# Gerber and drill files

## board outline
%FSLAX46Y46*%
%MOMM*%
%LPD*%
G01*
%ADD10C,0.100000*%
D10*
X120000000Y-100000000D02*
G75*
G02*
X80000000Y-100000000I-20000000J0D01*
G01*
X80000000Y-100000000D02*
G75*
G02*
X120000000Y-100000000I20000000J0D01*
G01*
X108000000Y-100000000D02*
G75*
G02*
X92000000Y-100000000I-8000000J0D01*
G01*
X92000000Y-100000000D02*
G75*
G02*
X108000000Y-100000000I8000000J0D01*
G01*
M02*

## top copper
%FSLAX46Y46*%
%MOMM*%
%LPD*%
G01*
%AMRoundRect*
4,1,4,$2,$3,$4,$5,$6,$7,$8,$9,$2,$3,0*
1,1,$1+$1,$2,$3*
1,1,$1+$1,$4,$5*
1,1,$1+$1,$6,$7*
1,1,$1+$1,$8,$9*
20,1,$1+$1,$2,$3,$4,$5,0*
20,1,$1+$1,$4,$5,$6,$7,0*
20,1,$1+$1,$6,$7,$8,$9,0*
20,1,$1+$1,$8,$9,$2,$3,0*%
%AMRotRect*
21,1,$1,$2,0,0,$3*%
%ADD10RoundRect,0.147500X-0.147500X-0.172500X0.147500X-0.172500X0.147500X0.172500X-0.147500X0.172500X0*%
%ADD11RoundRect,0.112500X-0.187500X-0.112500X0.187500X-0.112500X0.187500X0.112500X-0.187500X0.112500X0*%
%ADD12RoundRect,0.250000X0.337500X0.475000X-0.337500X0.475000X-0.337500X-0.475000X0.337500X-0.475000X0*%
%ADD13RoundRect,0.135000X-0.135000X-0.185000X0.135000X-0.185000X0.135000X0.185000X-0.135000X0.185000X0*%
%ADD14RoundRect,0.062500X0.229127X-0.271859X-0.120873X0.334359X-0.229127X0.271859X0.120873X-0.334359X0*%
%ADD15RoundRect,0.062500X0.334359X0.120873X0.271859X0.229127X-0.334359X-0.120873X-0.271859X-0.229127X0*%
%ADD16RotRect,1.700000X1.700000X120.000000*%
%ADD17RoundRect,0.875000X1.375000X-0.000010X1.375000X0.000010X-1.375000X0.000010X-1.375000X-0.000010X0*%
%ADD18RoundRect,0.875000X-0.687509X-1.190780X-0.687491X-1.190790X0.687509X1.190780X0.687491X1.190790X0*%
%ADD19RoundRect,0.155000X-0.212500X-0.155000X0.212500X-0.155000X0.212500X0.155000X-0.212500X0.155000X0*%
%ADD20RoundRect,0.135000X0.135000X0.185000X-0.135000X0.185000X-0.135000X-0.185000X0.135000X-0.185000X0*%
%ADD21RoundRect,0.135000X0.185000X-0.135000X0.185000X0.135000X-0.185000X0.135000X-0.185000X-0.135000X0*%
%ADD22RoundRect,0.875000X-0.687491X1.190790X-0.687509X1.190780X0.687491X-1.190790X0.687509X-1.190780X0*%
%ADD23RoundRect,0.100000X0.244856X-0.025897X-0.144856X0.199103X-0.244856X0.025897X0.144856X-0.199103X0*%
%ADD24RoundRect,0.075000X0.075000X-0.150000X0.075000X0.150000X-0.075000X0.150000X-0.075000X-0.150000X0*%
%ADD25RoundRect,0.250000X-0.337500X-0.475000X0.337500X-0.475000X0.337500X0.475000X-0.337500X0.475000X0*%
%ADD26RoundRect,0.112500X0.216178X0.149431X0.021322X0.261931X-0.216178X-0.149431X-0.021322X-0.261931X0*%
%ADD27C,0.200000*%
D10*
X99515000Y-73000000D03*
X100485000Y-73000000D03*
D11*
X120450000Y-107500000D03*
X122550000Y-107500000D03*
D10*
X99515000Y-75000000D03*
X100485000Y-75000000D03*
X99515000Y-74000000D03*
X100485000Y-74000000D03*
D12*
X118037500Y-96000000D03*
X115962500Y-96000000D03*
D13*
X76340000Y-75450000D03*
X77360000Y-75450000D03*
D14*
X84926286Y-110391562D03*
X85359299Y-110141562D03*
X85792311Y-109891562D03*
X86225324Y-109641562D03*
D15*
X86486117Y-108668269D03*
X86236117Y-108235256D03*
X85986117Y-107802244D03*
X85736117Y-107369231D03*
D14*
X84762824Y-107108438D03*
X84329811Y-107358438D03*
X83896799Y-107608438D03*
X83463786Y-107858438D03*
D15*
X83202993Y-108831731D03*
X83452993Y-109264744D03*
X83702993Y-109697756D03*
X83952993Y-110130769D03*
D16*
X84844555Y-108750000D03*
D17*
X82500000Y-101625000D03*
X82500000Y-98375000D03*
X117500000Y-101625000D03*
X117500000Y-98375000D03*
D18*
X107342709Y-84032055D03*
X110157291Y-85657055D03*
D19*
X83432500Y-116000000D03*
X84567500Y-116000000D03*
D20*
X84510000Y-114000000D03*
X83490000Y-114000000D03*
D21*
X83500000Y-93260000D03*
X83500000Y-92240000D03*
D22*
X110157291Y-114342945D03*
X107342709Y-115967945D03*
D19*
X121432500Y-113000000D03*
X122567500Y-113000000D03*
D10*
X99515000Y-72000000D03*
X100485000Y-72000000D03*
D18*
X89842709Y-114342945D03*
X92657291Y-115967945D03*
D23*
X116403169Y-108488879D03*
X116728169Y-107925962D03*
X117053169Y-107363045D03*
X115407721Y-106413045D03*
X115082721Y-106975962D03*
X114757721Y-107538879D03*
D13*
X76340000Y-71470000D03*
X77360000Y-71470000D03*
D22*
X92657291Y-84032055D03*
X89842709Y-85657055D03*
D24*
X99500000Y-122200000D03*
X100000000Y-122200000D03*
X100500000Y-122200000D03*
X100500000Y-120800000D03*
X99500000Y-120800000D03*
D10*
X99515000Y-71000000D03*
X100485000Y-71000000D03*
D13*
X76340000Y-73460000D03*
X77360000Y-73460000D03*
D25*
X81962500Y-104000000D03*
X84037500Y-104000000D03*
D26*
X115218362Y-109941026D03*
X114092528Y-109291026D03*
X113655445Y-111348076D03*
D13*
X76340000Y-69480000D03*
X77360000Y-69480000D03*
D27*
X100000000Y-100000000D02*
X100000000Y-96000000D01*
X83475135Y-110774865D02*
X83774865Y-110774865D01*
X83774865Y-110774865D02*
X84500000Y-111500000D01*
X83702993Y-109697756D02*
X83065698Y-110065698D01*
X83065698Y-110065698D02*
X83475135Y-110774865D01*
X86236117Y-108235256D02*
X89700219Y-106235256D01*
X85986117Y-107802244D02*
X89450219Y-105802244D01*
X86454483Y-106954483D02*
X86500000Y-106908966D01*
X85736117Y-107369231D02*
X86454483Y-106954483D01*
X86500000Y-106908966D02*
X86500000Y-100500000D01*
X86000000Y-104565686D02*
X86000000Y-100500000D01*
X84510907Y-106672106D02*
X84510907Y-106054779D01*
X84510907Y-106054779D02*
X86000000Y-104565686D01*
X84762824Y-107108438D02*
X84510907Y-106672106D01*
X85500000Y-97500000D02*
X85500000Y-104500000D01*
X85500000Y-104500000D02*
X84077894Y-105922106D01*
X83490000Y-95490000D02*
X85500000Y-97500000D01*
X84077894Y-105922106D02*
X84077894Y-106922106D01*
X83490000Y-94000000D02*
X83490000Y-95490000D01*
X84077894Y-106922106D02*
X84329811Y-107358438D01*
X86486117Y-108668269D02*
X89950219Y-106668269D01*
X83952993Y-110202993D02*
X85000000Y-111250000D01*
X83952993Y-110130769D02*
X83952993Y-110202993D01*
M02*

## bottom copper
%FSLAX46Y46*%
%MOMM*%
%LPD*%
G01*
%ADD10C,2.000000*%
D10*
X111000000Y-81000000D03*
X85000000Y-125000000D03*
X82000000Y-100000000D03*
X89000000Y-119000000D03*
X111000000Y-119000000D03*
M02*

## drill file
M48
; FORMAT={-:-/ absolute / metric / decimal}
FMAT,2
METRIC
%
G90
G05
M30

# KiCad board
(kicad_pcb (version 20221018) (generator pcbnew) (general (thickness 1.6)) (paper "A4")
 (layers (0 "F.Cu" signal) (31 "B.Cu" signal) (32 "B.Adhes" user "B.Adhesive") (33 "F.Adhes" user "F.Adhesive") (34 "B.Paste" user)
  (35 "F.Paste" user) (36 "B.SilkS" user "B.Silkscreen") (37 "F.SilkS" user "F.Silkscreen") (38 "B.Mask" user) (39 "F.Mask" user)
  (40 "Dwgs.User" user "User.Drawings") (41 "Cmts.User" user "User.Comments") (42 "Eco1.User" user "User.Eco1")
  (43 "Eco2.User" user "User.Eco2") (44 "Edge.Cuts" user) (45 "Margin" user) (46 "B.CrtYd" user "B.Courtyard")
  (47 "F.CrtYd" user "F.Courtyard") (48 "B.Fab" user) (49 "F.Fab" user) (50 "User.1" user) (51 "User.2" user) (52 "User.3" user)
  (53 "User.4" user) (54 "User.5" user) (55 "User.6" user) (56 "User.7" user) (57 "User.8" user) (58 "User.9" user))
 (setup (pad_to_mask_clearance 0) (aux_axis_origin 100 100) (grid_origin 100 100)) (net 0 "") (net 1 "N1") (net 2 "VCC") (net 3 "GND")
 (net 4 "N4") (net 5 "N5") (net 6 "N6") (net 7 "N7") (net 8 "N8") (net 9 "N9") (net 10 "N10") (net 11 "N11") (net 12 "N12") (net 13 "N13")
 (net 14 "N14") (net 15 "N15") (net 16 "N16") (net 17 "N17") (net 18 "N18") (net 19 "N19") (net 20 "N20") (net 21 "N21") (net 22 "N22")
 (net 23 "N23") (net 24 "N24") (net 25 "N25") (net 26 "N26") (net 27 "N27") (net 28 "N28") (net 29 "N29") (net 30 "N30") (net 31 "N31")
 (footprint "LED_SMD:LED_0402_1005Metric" (layer "F.Cu") (at 100 73)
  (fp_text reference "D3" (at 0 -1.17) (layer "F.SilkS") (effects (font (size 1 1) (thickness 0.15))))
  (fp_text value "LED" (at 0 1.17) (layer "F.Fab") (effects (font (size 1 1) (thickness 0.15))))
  (pad "1" smd roundrect (at -0.485 0) (size 0.59 0.64) (layers "F.Cu" "F.Paste" "F.Mask") (roundrect_rratio 0.25) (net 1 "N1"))
  (pad "2" smd roundrect (at 0.485 0) (size 0.59 0.64) (layers "F.Cu" "F.Paste" "F.Mask") (roundrect_rratio 0.25) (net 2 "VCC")))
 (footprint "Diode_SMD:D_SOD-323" (layer "F.Cu") (at 121.5 107.5)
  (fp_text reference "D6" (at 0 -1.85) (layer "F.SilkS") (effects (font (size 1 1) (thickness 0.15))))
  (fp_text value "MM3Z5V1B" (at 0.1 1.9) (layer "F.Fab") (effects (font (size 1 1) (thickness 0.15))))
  (pad "1" smd roundrect (at -1.05 0) (size 0.6 0.45) (layers "F.Cu" "F.Paste" "F.Mask") (roundrect_rratio 0.25) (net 2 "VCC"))
  (pad "2" smd roundrect (at 1.05 0) (size 0.6 0.45) (layers "F.Cu" "F.Paste" "F.Mask") (roundrect_rratio 0.25) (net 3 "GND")))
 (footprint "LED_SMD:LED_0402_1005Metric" (layer "F.Cu") (at 100 75)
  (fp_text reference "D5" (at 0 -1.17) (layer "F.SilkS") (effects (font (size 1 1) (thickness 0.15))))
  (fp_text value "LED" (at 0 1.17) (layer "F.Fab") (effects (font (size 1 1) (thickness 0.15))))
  (pad "1" smd roundrect (at -0.485 0) (size 0.59 0.64) (layers "F.Cu" "F.Paste" "F.Mask") (roundrect_rratio 0.25) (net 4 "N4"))
  (pad "2" smd roundrect (at 0.485 0) (size 0.59 0.64) (layers "F.Cu" "F.Paste" "F.Mask") (roundrect_rratio 0.25) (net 2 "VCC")))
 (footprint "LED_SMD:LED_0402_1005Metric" (layer "F.Cu") (at 100 74)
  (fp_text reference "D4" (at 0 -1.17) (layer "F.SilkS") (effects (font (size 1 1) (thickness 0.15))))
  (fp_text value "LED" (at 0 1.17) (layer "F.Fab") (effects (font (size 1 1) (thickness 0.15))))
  (pad "1" smd roundrect (at -0.485 0) (size 0.59 0.64) (layers "F.Cu" "F.Paste" "F.Mask") (roundrect_rratio 0.25) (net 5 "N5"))
  (pad "2" smd roundrect (at 0.485 0) (size 0.59 0.64) (layers "F.Cu" "F.Paste" "F.Mask") (roundrect_rratio 0.25) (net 2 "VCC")))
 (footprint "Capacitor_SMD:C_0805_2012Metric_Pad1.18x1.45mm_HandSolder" (layer "F.Cu") (at 117 96 180)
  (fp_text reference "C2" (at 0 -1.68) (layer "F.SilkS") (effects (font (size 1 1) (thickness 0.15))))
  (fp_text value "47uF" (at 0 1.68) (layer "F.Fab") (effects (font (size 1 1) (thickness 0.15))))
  (pad "1" smd roundrect (at -1.0375 0 180) (size 1.175 1.45) (layers "F.Cu" "F.Paste" "F.Mask") (roundrect_rratio 0.212766) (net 2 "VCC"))
  (pad "2" smd roundrect (at 1.0375 0 180) (size 1.175 1.45) (layers "F.Cu" "F.Paste" "F.Mask") (roundrect_rratio 0.212766) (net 3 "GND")))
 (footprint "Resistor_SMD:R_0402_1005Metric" (layer "F.Cu") (at 76.85 75.45)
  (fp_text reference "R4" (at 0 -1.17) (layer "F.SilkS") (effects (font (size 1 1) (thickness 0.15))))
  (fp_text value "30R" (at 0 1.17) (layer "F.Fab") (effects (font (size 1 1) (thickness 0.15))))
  (pad "1" smd roundrect (at -0.51 0) (size 0.54 0.64) (layers "F.Cu" "F.Paste" "F.Mask") (roundrect_rratio 0.25) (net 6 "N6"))
  (pad "2" smd roundrect (at 0.51 0) (size 0.54 0.64) (layers "F.Cu" "F.Paste" "F.Mask") (roundrect_rratio 0.25) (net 5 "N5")))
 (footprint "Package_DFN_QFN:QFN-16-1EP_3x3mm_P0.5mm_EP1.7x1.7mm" (layer "F.Cu") (at 84.844555 108.75 120)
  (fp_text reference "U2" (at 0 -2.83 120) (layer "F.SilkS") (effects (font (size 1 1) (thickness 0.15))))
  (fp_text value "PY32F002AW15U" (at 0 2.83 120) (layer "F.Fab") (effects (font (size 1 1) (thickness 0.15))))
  (pad "" smd roundrect (at -0.425 -0.425 120) (size 0.69 0.69) (layers "F.Paste") (roundrect_rratio 0.25))
  (pad "" smd roundrect (at -0.425 0.425 120) (size 0.69 0.69) (layers "F.Paste") (roundrect_rratio 0.25))
  (pad "" smd roundrect (at 0.425 -0.425 120) (size 0.69 0.69) (layers "F.Paste") (roundrect_rratio 0.25))
  (pad "" smd roundrect (at 0.425 0.425 120) (size 0.69 0.69) (layers "F.Paste") (roundrect_rratio 0.25))
  (pad "1" smd roundrect (at -1.4625 -0.75 120) (size 0.825 0.25) (layers "F.Cu" "F.Paste" "F.Mask") (roundrect_rratio 0.25) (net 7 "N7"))
  (pad "2" smd roundrect (at -1.4625 -0.25 120) (size 0.825 0.25) (layers "F.Cu" "F.Paste" "F.Mask") (roundrect_rratio 0.25) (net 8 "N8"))
  (pad "3" smd roundrect (at -1.4625 0.25 120) (size 0.825 0.25) (layers "F.Cu" "F.Paste" "F.Mask") (roundrect_rratio 0.25) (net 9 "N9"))
  (pad "4" smd roundrect (at -1.4625 0.75 120) (size 0.825 0.25) (layers "F.Cu" "F.Paste" "F.Mask") (roundrect_rratio 0.25) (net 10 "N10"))
  (pad "5" smd roundrect (at -0.75 1.4625 120) (size 0.25 0.825) (layers "F.Cu" "F.Paste" "F.Mask") (roundrect_rratio 0.25) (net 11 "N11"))
  (pad "6" smd roundrect (at -0.25 1.4625 120) (size 0.25 0.825) (layers "F.Cu" "F.Paste" "F.Mask") (roundrect_rratio 0.25) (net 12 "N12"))
  (pad "7" smd roundrect (at 0.25 1.4625 120) (size 0.25 0.825) (layers "F.Cu" "F.Paste" "F.Mask") (roundrect_rratio 0.25) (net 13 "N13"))
  (pad "8" smd roundrect (at 0.75 1.4625 120) (size 0.25 0.825) (layers "F.Cu" "F.Paste" "F.Mask") (roundrect_rratio 0.25) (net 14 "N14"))
  (pad "9" smd roundrect (at 1.4625 0.75 120) (size 0.825 0.25) (layers "F.Cu" "F.Paste" "F.Mask") (roundrect_rratio 0.25) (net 6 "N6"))
  (pad "10" smd roundrect (at 1.4625 0.25 120) (size 0.825 0.25) (layers "F.Cu" "F.Paste" "F.Mask") (roundrect_rratio 0.25) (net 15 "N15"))
  (pad "11" smd roundrect (at 1.4625 -0.25 120) (size 0.825 0.25) (layers "F.Cu" "F.Paste" "F.Mask") (roundrect_rratio 0.25) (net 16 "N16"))
  (pad "12" smd roundrect (at 1.4625 -0.75 120) (size 0.825 0.25) (layers "F.Cu" "F.Paste" "F.Mask") (roundrect_rratio 0.25) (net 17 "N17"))
  (pad "13" smd roundrect (at 0.75 -1.4625 120) (size 0.25 0.825) (layers "F.Cu" "F.Paste" "F.Mask") (roundrect_rratio 0.25) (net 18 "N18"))
  (pad "14" smd roundrect (at 0.25 -1.4625 120) (size 0.25 0.825) (layers "F.Cu" "F.Paste" "F.Mask") (roundrect_rratio 0.25) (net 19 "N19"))
  (pad "15" smd roundrect (at -0.25 -1.4625 120) (size 0.25 0.825) (layers "F.Cu" "F.Paste" "F.Mask") (roundrect_rratio 0.25) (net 2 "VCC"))
  (pad "16" smd roundrect (at -0.75 -1.4625 120) (size 0.25 0.825) (layers "F.Cu" "F.Paste" "F.Mask") (roundrect_rratio 0.25) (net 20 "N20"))
  (pad "17" smd rect (at 0 0 120) (size 1.7 1.7) (layers "F.Cu" "F.Mask") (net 3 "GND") (zone_connect 2)))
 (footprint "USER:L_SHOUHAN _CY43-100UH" (layer "F.Cu") (at 82.5 100 90)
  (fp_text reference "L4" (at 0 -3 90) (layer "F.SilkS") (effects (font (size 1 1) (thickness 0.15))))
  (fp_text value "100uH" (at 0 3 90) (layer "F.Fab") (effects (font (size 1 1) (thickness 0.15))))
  (pad "1" smd roundrect (at -1.625 0 90) (size 1.75 4.5) (layers "F.Cu" "F.Paste" "F.Mask") (roundrect_rratio 0.5) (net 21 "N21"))
  (pad "2" smd roundrect (at 1.625 0 90) (size 1.75 4.5) (layers "F.Cu" "F.Paste" "F.Mask") (roundrect_rratio 0.5) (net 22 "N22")))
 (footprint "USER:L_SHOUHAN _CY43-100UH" (layer "F.Cu") (at 117.5 100 90)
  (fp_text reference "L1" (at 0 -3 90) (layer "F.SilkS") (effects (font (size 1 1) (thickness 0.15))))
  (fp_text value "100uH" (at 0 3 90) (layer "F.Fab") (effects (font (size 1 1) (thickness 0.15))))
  (pad "1" smd roundrect (at -1.625 0 90) (size 1.75 4.5) (layers "F.Cu" "F.Paste" "F.Mask") (roundrect_rratio 0.5) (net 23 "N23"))
  (pad "2" smd roundrect (at 1.625 0 90) (size 1.75 4.5) (layers "F.Cu" "F.Paste" "F.Mask") (roundrect_rratio 0.5) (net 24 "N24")))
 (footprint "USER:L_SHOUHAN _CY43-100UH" (layer "F.Cu") (at 108.75 84.844555 -30)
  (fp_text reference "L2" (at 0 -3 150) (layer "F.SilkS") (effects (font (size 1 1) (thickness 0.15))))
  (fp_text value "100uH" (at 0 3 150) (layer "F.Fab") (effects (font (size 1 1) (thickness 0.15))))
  (pad "1" smd roundrect (at -1.625 0 330) (size 1.75 4.5) (layers "F.Cu" "F.Paste" "F.Mask") (roundrect_rratio 0.5) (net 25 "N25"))
  (pad "2" smd roundrect (at 1.625 0 330) (size 1.75 4.5) (layers "F.Cu" "F.Paste" "F.Mask") (roundrect_rratio 0.5) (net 24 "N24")))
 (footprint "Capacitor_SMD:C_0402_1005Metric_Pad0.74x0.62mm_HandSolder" (layer "F.Cu") (at 84 116)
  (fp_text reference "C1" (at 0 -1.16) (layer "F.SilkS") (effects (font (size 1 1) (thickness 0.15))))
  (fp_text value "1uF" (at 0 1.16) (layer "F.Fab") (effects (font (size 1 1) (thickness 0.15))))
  (pad "1" smd roundrect (at -0.5675 0) (size 0.735 0.62) (layers "F.Cu" "F.Paste" "F.Mask") (roundrect_rratio 0.25) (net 2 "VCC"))
  (pad "2" smd roundrect (at 0.5675 0) (size 0.735 0.62) (layers "F.Cu" "F.Paste" "F.Mask") (roundrect_rratio 0.25) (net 3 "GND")))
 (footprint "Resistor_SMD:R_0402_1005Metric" (layer "F.Cu") (at 84 114 180)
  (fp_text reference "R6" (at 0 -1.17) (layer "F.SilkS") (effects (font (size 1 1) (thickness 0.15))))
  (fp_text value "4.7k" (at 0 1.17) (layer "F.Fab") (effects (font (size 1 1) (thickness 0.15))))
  (pad "1" smd roundrect (at -0.51 0 180) (size 0.54 0.64) (layers "F.Cu" "F.Paste" "F.Mask") (roundrect_rratio 0.25) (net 11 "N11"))
  (pad "2" smd roundrect (at 0.51 0 180) (size 0.54 0.64) (layers "F.Cu" "F.Paste" "F.Mask") (roundrect_rratio 0.25) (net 2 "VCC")))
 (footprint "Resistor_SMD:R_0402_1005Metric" (layer "F.Cu") (at 83.5 92.75 90)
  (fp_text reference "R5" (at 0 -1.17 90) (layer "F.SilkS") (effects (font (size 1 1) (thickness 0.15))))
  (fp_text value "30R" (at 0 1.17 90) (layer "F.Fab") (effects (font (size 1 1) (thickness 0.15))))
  (pad "1" smd roundrect (at -0.51 0 90) (size 0.54 0.64) (layers "F.Cu" "F.Paste" "F.Mask") (roundrect_rratio 0.25) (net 15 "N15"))
  (pad "2" smd roundrect (at 0.51 0 90) (size 0.54 0.64) (layers "F.Cu" "F.Paste" "F.Mask") (roundrect_rratio 0.25) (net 4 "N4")))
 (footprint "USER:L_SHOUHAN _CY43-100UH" (layer "F.Cu") (at 108.75 115.155445 -150)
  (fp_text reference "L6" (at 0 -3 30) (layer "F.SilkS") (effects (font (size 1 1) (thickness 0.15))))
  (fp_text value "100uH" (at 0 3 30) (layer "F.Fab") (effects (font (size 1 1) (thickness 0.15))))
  (pad "1" smd roundrect (at -1.625 0 210) (size 1.75 4.5) (layers "F.Cu" "F.Paste" "F.Mask") (roundrect_rratio 0.5) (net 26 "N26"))
  (pad "2" smd roundrect (at 1.625 0 210) (size 1.75 4.5) (layers "F.Cu" "F.Paste" "F.Mask") (roundrect_rratio 0.5) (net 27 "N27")))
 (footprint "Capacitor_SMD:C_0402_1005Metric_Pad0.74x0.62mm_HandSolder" (layer "F.Cu") (at 122 113)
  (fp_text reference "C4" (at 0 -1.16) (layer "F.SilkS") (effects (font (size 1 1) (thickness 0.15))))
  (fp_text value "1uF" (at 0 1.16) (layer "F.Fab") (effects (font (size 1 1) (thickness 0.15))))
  (pad "1" smd roundrect (at -0.5675 0) (size 0.735 0.62) (layers "F.Cu" "F.Paste" "F.Mask") (roundrect_rratio 0.25) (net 2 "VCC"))
  (pad "2" smd roundrect (at 0.5675 0) (size 0.735 0.62) (layers "F.Cu" "F.Paste" "F.Mask") (roundrect_rratio 0.25) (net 3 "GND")))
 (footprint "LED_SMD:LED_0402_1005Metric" (layer "F.Cu") (at 100 72)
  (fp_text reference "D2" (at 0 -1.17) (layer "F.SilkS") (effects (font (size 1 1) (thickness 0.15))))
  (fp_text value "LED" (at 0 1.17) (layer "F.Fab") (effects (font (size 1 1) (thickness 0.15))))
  (pad "1" smd roundrect (at -0.485 0) (size 0.59 0.64) (layers "F.Cu" "F.Paste" "F.Mask") (roundrect_rratio 0.25) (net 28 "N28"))
  (pad "2" smd roundrect (at 0.485 0) (size 0.59 0.64) (layers "F.Cu" "F.Paste" "F.Mask") (roundrect_rratio 0.25) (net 2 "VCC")))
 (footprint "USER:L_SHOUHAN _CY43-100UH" (layer "F.Cu") (at 91.25 115.155445 -30)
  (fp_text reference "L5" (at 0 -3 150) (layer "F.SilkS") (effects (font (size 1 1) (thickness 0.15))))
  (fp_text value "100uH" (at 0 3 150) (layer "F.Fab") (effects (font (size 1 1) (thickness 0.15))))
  (pad "1" smd roundrect (at -1.625 0 330) (size 1.75 4.5) (layers "F.Cu" "F.Paste" "F.Mask") (roundrect_rratio 0.5) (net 21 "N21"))
  (pad "2" smd roundrect (at 1.625 0 330) (size 1.75 4.5) (layers "F.Cu" "F.Paste" "F.Mask") (roundrect_rratio 0.5) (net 27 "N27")))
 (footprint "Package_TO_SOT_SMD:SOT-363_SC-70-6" (layer "F.Cu") (at 115.905445 107.450962 150)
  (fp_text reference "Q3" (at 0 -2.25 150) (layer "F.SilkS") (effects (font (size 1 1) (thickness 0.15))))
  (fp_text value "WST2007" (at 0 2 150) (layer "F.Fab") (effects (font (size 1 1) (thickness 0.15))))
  (pad "1" smd roundrect (at -0.95 -0.65 150) (size 0.65 0.4) (layers "F.Cu" "F.Paste" "F.Mask") (roundrect_rratio 0.25) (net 3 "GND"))
  (pad "2" smd roundrect (at -0.95 0 150) (size 0.65 0.4) (layers "F.Cu" "F.Paste" "F.Mask") (roundrect_rratio 0.25) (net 26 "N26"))
  (pad "3" smd roundrect (at -0.95 0.65 150) (size 0.65 0.4) (layers "F.Cu" "F.Paste" "F.Mask") (roundrect_rratio 0.25) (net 26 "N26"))
  (pad "4" smd roundrect (at 0.95 0.65 150) (size 0.65 0.4) (layers "F.Cu" "F.Paste" "F.Mask") (roundrect_rratio 0.25) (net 3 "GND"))
  (pad "5" smd roundrect (at 0.95 0 150) (size 0.65 0.4) (layers "F.Cu" "F.Paste" "F.Mask") (roundrect_rratio 0.25) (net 23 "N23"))
  (pad "6" smd roundrect (at 0.95 -0.65 150) (size 0.65 0.4) (layers "F.Cu" "F.Paste" "F.Mask") (roundrect_rratio 0.25) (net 23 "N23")))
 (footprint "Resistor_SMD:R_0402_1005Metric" (layer "F.Cu") (at 76.85 71.47)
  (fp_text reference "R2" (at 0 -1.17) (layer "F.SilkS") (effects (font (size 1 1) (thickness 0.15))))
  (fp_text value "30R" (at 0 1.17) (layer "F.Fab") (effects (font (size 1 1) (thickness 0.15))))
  (pad "1" smd roundrect (at -0.51 0) (size 0.54 0.64) (layers "F.Cu" "F.Paste" "F.Mask") (roundrect_rratio 0.25) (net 13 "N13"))
  (pad "2" smd roundrect (at 0.51 0) (size 0.54 0.64) (layers "F.Cu" "F.Paste" "F.Mask") (roundrect_rratio 0.25) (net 28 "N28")))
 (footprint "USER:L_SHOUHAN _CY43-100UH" (layer "F.Cu") (at 91.25 84.844555 -150)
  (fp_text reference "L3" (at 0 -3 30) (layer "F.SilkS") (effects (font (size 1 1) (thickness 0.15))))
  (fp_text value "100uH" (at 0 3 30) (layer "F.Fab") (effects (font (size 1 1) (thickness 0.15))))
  (pad "1" smd roundrect (at -1.625 0 210) (size 1.75 4.5) (layers "F.Cu" "F.Paste" "F.Mask") (roundrect_rratio 0.5) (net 25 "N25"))
  (pad "2" smd roundrect (at 1.625 0 210) (size 1.75 4.5) (layers "F.Cu" "F.Paste" "F.Mask") (roundrect_rratio 0.5) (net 22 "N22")))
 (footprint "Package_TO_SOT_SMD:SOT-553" (layer "F.Cu") (at 100 121.5 90)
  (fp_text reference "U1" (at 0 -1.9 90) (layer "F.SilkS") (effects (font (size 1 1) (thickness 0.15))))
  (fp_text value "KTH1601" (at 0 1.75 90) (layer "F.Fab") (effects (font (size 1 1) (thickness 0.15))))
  (pad "1" smd roundrect (at -0.7 -0.5 90) (size 0.45 0.3) (layers "F.Cu" "F.Paste" "F.Mask") (roundrect_rratio 0.25) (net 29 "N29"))
  (pad "2" smd roundrect (at -0.7 0 90) (size 0.45 0.3) (layers "F.Cu" "F.Paste" "F.Mask") (roundrect_rratio 0.25) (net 3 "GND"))
  (pad "3" smd roundrect (at -0.7 0.5 90) (size 0.45 0.3) (layers "F.Cu" "F.Paste" "F.Mask") (roundrect_rratio 0.25) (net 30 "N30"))
  (pad "4" smd roundrect (at 0.7 0.5 90) (size 0.45 0.3) (layers "F.Cu" "F.Paste" "F.Mask") (roundrect_rratio 0.25) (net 2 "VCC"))
  (pad "5" smd roundrect (at 0.7 -0.5 90) (size 0.45 0.3) (layers "F.Cu" "F.Paste" "F.Mask") (roundrect_rratio 0.25) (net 20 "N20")))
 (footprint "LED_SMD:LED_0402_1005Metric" (layer "F.Cu") (at 100 71)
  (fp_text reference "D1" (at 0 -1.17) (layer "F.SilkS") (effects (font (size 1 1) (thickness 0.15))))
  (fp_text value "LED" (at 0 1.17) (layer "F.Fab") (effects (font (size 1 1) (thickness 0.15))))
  (pad "1" smd roundrect (at -0.485 0) (size 0.59 0.64) (layers "F.Cu" "F.Paste" "F.Mask") (roundrect_rratio 0.25) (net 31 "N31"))
  (pad "2" smd roundrect (at 0.485 0) (size 0.59 0.64) (layers "F.Cu" "F.Paste" "F.Mask") (roundrect_rratio 0.25) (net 2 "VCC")))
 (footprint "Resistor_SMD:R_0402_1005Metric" (layer "F.Cu") (at 76.85 73.46)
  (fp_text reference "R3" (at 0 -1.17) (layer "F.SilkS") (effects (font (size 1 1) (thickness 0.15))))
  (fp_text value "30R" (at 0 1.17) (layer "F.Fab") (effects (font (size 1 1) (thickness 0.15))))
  (pad "1" smd roundrect (at -0.51 0) (size 0.54 0.64) (layers "F.Cu" "F.Paste" "F.Mask") (roundrect_rratio 0.25) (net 14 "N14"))
  (pad "2" smd roundrect (at 0.51 0) (size 0.54 0.64) (layers "F.Cu" "F.Paste" "F.Mask") (roundrect_rratio 0.25) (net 1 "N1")))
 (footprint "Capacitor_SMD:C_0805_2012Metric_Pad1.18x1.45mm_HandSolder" (layer "F.Cu") (at 83 104)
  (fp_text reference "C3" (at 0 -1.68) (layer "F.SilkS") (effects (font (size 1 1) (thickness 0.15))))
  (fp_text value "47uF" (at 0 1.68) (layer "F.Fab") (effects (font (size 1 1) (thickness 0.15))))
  (pad "1" smd roundrect (at -1.0375 0) (size 1.175 1.45) (layers "F.Cu" "F.Paste" "F.Mask") (roundrect_rratio 0.212766) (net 2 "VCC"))
  (pad "2" smd roundrect (at 1.0375 0) (size 1.175 1.45) (layers "F.Cu" "F.Paste" "F.Mask") (roundrect_rratio 0.212766) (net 3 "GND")))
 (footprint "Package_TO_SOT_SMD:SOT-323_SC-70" (layer "F.Cu") (at 114.155445 110.482051 -120)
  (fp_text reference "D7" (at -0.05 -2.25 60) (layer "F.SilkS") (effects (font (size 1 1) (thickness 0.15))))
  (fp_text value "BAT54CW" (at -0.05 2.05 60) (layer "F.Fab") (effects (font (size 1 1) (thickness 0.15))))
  (pad "1" smd roundrect (at -1 -0.65 150) (size 0.45 0.7) (layers "F.Cu" "F.Paste" "F.Mask") (roundrect_rratio 0.25) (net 26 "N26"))
  (pad "2" smd roundrect (at -1 0.65 150) (size 0.45 0.7) (layers "F.Cu" "F.Paste" "F.Mask") (roundrect_rratio 0.25) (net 23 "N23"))
  (pad "3" smd roundrect (at 1 0 150) (size 0.45 0.7) (layers "F.Cu" "F.Paste" "F.Mask") (roundrect_rratio 0.25) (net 2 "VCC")))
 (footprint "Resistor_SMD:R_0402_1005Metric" (layer "F.Cu") (at 76.85 69.48)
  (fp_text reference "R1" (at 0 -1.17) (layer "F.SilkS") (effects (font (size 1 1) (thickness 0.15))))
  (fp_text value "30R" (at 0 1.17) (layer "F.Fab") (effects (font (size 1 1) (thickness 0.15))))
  (pad "1" smd roundrect (at -0.51 0) (size 0.54 0.64) (layers "F.Cu" "F.Paste" "F.Mask") (roundrect_rratio 0.25) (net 12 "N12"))
  (pad "2" smd roundrect (at 0.51 0) (size 0.54 0.64) (layers "F.Cu" "F.Paste" "F.Mask") (roundrect_rratio 0.25) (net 31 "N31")))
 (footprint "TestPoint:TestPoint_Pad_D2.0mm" (layer "B.Cu") (at 111 81 180)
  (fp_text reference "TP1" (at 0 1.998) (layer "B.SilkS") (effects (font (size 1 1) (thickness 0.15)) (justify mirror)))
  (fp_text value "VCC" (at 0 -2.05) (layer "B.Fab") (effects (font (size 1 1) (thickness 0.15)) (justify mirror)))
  (pad "1" smd circle (at 0 0 180) (size 2 2) (layers "B.Cu" "B.Mask") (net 2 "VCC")))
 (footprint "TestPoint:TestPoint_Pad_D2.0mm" (layer "B.Cu") (at 85 125 180)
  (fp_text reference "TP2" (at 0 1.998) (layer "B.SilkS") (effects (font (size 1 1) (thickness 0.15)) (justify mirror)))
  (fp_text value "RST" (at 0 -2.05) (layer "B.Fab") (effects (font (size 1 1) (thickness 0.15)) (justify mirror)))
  (pad "1" smd circle (at 0 0 180) (size 2 2) (layers "B.Cu" "B.Mask") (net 11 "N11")))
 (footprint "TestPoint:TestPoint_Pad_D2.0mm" (layer "B.Cu") (at 82 100 180)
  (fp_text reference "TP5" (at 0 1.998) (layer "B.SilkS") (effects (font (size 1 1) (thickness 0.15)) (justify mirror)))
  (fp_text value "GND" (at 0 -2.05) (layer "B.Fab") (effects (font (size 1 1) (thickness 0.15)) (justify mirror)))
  (pad "1" smd circle (at 0 0 180) (size 2 2) (layers "B.Cu" "B.Mask") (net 3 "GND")))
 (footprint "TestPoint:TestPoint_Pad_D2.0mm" (layer "B.Cu") (at 89 119 180)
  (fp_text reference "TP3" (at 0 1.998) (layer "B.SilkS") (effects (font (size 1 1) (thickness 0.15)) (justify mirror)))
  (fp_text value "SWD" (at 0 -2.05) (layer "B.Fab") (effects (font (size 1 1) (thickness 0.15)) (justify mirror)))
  (pad "1" smd circle (at 0 0 180) (size 2 2) (layers "B.Cu" "B.Mask") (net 9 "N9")))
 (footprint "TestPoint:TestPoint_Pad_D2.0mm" (layer "B.Cu") (at 111 119 180)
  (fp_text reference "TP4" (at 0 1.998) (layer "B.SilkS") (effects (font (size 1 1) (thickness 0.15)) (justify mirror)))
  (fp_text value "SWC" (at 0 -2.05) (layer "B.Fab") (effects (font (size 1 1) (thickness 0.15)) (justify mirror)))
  (pad "1" smd circle (at 0 0 180) (size 2 2) (layers "B.Cu" "B.Mask") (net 10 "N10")))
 (gr_circle (center 100 100) (end 100 80) (stroke (width 0.1) (type default)) (fill none) (layer "Edge.Cuts"))
 (gr_circle locked (center 100 100) (end 108 100) (stroke (width 0.1) (type default)) (fill none) (layer "Edge.Cuts"))
 (segment (start 100 100) (end 100 96) (width 0.2) (layer "F.Cu") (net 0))
 (segment (start 83.475135 110.774865) (end 83.774865 110.774865) (width 0.2) (layer "F.Cu") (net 2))
 (segment (start 83.774865 110.774865) (end 84.5 111.5) (width 0.2) (layer "F.Cu") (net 2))
 (segment (start 83.702993 109.697756) (end 83.065698 110.065698) (width 0.2) (layer "F.Cu") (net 2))
 (segment (start 83.065698 110.065698) (end 83.475135 110.774865) (width 0.2) (layer "F.Cu") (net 2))
 (segment (start 86.236117 108.235256) (end 89.700219 106.235256) (width 0.2) (layer "F.Cu") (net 12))
 (segment (start 85.986117 107.802244) (end 89.450219 105.802244) (width 0.2) (layer "F.Cu") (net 13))
 (segment (start 86.454483 106.954483) (end 86.5 106.908966) (width 0.2) (layer "F.Cu") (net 14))
 (segment (start 85.736117 107.369231) (end 86.454483 106.954483) (width 0.2) (layer "F.Cu") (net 14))
 (segment (start 86.5 106.908966) (end 86.5 100.5) (width 0.2) (layer "F.Cu") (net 14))
 (segment (start 86 104.565686) (end 86 100.5) (width 0.2) (layer "F.Cu") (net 6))
 (segment (start 84.510907 106.672106) (end 84.510907 106.054779) (width 0.2) (layer "F.Cu") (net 6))
 (segment (start 84.510907 106.054779) (end 86 104.565686) (width 0.2) (layer "F.Cu") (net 6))
 (segment (start 84.762824 107.108438) (end 84.510907 106.672106) (width 0.2) (layer "F.Cu") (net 6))
 (segment (start 85.5 97.5) (end 85.5 104.5) (width 0.2) (layer "F.Cu") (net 15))
 (segment (start 85.5 104.5) (end 84.077894 105.922106) (width 0.2) (layer "F.Cu") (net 15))
 (segment (start 83.49 95.49) (end 85.5 97.5) (width 0.2) (layer "F.Cu") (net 15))
 (segment (start 84.077894 105.922106) (end 84.077894 106.922106) (width 0.2) (layer "F.Cu") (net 15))
 (segment (start 83.49 94) (end 83.49 95.49) (width 0.2) (layer "F.Cu") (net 15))
 (segment (start 84.077894 106.922106) (end 84.329811 107.358438) (width 0.2) (layer "F.Cu") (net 15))
 (segment (start 86.486117 108.668269) (end 89.950219 106.668269) (width 0.2) (layer "F.Cu") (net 11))
 (segment (start 83.952993 110.202993) (end 85 111.25) (width 0.2) (layer "F.Cu") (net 20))
 (segment (start 83.952993 110.130769) (end 83.952993 110.202993) (width 0.2) (layer "F.Cu") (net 20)))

